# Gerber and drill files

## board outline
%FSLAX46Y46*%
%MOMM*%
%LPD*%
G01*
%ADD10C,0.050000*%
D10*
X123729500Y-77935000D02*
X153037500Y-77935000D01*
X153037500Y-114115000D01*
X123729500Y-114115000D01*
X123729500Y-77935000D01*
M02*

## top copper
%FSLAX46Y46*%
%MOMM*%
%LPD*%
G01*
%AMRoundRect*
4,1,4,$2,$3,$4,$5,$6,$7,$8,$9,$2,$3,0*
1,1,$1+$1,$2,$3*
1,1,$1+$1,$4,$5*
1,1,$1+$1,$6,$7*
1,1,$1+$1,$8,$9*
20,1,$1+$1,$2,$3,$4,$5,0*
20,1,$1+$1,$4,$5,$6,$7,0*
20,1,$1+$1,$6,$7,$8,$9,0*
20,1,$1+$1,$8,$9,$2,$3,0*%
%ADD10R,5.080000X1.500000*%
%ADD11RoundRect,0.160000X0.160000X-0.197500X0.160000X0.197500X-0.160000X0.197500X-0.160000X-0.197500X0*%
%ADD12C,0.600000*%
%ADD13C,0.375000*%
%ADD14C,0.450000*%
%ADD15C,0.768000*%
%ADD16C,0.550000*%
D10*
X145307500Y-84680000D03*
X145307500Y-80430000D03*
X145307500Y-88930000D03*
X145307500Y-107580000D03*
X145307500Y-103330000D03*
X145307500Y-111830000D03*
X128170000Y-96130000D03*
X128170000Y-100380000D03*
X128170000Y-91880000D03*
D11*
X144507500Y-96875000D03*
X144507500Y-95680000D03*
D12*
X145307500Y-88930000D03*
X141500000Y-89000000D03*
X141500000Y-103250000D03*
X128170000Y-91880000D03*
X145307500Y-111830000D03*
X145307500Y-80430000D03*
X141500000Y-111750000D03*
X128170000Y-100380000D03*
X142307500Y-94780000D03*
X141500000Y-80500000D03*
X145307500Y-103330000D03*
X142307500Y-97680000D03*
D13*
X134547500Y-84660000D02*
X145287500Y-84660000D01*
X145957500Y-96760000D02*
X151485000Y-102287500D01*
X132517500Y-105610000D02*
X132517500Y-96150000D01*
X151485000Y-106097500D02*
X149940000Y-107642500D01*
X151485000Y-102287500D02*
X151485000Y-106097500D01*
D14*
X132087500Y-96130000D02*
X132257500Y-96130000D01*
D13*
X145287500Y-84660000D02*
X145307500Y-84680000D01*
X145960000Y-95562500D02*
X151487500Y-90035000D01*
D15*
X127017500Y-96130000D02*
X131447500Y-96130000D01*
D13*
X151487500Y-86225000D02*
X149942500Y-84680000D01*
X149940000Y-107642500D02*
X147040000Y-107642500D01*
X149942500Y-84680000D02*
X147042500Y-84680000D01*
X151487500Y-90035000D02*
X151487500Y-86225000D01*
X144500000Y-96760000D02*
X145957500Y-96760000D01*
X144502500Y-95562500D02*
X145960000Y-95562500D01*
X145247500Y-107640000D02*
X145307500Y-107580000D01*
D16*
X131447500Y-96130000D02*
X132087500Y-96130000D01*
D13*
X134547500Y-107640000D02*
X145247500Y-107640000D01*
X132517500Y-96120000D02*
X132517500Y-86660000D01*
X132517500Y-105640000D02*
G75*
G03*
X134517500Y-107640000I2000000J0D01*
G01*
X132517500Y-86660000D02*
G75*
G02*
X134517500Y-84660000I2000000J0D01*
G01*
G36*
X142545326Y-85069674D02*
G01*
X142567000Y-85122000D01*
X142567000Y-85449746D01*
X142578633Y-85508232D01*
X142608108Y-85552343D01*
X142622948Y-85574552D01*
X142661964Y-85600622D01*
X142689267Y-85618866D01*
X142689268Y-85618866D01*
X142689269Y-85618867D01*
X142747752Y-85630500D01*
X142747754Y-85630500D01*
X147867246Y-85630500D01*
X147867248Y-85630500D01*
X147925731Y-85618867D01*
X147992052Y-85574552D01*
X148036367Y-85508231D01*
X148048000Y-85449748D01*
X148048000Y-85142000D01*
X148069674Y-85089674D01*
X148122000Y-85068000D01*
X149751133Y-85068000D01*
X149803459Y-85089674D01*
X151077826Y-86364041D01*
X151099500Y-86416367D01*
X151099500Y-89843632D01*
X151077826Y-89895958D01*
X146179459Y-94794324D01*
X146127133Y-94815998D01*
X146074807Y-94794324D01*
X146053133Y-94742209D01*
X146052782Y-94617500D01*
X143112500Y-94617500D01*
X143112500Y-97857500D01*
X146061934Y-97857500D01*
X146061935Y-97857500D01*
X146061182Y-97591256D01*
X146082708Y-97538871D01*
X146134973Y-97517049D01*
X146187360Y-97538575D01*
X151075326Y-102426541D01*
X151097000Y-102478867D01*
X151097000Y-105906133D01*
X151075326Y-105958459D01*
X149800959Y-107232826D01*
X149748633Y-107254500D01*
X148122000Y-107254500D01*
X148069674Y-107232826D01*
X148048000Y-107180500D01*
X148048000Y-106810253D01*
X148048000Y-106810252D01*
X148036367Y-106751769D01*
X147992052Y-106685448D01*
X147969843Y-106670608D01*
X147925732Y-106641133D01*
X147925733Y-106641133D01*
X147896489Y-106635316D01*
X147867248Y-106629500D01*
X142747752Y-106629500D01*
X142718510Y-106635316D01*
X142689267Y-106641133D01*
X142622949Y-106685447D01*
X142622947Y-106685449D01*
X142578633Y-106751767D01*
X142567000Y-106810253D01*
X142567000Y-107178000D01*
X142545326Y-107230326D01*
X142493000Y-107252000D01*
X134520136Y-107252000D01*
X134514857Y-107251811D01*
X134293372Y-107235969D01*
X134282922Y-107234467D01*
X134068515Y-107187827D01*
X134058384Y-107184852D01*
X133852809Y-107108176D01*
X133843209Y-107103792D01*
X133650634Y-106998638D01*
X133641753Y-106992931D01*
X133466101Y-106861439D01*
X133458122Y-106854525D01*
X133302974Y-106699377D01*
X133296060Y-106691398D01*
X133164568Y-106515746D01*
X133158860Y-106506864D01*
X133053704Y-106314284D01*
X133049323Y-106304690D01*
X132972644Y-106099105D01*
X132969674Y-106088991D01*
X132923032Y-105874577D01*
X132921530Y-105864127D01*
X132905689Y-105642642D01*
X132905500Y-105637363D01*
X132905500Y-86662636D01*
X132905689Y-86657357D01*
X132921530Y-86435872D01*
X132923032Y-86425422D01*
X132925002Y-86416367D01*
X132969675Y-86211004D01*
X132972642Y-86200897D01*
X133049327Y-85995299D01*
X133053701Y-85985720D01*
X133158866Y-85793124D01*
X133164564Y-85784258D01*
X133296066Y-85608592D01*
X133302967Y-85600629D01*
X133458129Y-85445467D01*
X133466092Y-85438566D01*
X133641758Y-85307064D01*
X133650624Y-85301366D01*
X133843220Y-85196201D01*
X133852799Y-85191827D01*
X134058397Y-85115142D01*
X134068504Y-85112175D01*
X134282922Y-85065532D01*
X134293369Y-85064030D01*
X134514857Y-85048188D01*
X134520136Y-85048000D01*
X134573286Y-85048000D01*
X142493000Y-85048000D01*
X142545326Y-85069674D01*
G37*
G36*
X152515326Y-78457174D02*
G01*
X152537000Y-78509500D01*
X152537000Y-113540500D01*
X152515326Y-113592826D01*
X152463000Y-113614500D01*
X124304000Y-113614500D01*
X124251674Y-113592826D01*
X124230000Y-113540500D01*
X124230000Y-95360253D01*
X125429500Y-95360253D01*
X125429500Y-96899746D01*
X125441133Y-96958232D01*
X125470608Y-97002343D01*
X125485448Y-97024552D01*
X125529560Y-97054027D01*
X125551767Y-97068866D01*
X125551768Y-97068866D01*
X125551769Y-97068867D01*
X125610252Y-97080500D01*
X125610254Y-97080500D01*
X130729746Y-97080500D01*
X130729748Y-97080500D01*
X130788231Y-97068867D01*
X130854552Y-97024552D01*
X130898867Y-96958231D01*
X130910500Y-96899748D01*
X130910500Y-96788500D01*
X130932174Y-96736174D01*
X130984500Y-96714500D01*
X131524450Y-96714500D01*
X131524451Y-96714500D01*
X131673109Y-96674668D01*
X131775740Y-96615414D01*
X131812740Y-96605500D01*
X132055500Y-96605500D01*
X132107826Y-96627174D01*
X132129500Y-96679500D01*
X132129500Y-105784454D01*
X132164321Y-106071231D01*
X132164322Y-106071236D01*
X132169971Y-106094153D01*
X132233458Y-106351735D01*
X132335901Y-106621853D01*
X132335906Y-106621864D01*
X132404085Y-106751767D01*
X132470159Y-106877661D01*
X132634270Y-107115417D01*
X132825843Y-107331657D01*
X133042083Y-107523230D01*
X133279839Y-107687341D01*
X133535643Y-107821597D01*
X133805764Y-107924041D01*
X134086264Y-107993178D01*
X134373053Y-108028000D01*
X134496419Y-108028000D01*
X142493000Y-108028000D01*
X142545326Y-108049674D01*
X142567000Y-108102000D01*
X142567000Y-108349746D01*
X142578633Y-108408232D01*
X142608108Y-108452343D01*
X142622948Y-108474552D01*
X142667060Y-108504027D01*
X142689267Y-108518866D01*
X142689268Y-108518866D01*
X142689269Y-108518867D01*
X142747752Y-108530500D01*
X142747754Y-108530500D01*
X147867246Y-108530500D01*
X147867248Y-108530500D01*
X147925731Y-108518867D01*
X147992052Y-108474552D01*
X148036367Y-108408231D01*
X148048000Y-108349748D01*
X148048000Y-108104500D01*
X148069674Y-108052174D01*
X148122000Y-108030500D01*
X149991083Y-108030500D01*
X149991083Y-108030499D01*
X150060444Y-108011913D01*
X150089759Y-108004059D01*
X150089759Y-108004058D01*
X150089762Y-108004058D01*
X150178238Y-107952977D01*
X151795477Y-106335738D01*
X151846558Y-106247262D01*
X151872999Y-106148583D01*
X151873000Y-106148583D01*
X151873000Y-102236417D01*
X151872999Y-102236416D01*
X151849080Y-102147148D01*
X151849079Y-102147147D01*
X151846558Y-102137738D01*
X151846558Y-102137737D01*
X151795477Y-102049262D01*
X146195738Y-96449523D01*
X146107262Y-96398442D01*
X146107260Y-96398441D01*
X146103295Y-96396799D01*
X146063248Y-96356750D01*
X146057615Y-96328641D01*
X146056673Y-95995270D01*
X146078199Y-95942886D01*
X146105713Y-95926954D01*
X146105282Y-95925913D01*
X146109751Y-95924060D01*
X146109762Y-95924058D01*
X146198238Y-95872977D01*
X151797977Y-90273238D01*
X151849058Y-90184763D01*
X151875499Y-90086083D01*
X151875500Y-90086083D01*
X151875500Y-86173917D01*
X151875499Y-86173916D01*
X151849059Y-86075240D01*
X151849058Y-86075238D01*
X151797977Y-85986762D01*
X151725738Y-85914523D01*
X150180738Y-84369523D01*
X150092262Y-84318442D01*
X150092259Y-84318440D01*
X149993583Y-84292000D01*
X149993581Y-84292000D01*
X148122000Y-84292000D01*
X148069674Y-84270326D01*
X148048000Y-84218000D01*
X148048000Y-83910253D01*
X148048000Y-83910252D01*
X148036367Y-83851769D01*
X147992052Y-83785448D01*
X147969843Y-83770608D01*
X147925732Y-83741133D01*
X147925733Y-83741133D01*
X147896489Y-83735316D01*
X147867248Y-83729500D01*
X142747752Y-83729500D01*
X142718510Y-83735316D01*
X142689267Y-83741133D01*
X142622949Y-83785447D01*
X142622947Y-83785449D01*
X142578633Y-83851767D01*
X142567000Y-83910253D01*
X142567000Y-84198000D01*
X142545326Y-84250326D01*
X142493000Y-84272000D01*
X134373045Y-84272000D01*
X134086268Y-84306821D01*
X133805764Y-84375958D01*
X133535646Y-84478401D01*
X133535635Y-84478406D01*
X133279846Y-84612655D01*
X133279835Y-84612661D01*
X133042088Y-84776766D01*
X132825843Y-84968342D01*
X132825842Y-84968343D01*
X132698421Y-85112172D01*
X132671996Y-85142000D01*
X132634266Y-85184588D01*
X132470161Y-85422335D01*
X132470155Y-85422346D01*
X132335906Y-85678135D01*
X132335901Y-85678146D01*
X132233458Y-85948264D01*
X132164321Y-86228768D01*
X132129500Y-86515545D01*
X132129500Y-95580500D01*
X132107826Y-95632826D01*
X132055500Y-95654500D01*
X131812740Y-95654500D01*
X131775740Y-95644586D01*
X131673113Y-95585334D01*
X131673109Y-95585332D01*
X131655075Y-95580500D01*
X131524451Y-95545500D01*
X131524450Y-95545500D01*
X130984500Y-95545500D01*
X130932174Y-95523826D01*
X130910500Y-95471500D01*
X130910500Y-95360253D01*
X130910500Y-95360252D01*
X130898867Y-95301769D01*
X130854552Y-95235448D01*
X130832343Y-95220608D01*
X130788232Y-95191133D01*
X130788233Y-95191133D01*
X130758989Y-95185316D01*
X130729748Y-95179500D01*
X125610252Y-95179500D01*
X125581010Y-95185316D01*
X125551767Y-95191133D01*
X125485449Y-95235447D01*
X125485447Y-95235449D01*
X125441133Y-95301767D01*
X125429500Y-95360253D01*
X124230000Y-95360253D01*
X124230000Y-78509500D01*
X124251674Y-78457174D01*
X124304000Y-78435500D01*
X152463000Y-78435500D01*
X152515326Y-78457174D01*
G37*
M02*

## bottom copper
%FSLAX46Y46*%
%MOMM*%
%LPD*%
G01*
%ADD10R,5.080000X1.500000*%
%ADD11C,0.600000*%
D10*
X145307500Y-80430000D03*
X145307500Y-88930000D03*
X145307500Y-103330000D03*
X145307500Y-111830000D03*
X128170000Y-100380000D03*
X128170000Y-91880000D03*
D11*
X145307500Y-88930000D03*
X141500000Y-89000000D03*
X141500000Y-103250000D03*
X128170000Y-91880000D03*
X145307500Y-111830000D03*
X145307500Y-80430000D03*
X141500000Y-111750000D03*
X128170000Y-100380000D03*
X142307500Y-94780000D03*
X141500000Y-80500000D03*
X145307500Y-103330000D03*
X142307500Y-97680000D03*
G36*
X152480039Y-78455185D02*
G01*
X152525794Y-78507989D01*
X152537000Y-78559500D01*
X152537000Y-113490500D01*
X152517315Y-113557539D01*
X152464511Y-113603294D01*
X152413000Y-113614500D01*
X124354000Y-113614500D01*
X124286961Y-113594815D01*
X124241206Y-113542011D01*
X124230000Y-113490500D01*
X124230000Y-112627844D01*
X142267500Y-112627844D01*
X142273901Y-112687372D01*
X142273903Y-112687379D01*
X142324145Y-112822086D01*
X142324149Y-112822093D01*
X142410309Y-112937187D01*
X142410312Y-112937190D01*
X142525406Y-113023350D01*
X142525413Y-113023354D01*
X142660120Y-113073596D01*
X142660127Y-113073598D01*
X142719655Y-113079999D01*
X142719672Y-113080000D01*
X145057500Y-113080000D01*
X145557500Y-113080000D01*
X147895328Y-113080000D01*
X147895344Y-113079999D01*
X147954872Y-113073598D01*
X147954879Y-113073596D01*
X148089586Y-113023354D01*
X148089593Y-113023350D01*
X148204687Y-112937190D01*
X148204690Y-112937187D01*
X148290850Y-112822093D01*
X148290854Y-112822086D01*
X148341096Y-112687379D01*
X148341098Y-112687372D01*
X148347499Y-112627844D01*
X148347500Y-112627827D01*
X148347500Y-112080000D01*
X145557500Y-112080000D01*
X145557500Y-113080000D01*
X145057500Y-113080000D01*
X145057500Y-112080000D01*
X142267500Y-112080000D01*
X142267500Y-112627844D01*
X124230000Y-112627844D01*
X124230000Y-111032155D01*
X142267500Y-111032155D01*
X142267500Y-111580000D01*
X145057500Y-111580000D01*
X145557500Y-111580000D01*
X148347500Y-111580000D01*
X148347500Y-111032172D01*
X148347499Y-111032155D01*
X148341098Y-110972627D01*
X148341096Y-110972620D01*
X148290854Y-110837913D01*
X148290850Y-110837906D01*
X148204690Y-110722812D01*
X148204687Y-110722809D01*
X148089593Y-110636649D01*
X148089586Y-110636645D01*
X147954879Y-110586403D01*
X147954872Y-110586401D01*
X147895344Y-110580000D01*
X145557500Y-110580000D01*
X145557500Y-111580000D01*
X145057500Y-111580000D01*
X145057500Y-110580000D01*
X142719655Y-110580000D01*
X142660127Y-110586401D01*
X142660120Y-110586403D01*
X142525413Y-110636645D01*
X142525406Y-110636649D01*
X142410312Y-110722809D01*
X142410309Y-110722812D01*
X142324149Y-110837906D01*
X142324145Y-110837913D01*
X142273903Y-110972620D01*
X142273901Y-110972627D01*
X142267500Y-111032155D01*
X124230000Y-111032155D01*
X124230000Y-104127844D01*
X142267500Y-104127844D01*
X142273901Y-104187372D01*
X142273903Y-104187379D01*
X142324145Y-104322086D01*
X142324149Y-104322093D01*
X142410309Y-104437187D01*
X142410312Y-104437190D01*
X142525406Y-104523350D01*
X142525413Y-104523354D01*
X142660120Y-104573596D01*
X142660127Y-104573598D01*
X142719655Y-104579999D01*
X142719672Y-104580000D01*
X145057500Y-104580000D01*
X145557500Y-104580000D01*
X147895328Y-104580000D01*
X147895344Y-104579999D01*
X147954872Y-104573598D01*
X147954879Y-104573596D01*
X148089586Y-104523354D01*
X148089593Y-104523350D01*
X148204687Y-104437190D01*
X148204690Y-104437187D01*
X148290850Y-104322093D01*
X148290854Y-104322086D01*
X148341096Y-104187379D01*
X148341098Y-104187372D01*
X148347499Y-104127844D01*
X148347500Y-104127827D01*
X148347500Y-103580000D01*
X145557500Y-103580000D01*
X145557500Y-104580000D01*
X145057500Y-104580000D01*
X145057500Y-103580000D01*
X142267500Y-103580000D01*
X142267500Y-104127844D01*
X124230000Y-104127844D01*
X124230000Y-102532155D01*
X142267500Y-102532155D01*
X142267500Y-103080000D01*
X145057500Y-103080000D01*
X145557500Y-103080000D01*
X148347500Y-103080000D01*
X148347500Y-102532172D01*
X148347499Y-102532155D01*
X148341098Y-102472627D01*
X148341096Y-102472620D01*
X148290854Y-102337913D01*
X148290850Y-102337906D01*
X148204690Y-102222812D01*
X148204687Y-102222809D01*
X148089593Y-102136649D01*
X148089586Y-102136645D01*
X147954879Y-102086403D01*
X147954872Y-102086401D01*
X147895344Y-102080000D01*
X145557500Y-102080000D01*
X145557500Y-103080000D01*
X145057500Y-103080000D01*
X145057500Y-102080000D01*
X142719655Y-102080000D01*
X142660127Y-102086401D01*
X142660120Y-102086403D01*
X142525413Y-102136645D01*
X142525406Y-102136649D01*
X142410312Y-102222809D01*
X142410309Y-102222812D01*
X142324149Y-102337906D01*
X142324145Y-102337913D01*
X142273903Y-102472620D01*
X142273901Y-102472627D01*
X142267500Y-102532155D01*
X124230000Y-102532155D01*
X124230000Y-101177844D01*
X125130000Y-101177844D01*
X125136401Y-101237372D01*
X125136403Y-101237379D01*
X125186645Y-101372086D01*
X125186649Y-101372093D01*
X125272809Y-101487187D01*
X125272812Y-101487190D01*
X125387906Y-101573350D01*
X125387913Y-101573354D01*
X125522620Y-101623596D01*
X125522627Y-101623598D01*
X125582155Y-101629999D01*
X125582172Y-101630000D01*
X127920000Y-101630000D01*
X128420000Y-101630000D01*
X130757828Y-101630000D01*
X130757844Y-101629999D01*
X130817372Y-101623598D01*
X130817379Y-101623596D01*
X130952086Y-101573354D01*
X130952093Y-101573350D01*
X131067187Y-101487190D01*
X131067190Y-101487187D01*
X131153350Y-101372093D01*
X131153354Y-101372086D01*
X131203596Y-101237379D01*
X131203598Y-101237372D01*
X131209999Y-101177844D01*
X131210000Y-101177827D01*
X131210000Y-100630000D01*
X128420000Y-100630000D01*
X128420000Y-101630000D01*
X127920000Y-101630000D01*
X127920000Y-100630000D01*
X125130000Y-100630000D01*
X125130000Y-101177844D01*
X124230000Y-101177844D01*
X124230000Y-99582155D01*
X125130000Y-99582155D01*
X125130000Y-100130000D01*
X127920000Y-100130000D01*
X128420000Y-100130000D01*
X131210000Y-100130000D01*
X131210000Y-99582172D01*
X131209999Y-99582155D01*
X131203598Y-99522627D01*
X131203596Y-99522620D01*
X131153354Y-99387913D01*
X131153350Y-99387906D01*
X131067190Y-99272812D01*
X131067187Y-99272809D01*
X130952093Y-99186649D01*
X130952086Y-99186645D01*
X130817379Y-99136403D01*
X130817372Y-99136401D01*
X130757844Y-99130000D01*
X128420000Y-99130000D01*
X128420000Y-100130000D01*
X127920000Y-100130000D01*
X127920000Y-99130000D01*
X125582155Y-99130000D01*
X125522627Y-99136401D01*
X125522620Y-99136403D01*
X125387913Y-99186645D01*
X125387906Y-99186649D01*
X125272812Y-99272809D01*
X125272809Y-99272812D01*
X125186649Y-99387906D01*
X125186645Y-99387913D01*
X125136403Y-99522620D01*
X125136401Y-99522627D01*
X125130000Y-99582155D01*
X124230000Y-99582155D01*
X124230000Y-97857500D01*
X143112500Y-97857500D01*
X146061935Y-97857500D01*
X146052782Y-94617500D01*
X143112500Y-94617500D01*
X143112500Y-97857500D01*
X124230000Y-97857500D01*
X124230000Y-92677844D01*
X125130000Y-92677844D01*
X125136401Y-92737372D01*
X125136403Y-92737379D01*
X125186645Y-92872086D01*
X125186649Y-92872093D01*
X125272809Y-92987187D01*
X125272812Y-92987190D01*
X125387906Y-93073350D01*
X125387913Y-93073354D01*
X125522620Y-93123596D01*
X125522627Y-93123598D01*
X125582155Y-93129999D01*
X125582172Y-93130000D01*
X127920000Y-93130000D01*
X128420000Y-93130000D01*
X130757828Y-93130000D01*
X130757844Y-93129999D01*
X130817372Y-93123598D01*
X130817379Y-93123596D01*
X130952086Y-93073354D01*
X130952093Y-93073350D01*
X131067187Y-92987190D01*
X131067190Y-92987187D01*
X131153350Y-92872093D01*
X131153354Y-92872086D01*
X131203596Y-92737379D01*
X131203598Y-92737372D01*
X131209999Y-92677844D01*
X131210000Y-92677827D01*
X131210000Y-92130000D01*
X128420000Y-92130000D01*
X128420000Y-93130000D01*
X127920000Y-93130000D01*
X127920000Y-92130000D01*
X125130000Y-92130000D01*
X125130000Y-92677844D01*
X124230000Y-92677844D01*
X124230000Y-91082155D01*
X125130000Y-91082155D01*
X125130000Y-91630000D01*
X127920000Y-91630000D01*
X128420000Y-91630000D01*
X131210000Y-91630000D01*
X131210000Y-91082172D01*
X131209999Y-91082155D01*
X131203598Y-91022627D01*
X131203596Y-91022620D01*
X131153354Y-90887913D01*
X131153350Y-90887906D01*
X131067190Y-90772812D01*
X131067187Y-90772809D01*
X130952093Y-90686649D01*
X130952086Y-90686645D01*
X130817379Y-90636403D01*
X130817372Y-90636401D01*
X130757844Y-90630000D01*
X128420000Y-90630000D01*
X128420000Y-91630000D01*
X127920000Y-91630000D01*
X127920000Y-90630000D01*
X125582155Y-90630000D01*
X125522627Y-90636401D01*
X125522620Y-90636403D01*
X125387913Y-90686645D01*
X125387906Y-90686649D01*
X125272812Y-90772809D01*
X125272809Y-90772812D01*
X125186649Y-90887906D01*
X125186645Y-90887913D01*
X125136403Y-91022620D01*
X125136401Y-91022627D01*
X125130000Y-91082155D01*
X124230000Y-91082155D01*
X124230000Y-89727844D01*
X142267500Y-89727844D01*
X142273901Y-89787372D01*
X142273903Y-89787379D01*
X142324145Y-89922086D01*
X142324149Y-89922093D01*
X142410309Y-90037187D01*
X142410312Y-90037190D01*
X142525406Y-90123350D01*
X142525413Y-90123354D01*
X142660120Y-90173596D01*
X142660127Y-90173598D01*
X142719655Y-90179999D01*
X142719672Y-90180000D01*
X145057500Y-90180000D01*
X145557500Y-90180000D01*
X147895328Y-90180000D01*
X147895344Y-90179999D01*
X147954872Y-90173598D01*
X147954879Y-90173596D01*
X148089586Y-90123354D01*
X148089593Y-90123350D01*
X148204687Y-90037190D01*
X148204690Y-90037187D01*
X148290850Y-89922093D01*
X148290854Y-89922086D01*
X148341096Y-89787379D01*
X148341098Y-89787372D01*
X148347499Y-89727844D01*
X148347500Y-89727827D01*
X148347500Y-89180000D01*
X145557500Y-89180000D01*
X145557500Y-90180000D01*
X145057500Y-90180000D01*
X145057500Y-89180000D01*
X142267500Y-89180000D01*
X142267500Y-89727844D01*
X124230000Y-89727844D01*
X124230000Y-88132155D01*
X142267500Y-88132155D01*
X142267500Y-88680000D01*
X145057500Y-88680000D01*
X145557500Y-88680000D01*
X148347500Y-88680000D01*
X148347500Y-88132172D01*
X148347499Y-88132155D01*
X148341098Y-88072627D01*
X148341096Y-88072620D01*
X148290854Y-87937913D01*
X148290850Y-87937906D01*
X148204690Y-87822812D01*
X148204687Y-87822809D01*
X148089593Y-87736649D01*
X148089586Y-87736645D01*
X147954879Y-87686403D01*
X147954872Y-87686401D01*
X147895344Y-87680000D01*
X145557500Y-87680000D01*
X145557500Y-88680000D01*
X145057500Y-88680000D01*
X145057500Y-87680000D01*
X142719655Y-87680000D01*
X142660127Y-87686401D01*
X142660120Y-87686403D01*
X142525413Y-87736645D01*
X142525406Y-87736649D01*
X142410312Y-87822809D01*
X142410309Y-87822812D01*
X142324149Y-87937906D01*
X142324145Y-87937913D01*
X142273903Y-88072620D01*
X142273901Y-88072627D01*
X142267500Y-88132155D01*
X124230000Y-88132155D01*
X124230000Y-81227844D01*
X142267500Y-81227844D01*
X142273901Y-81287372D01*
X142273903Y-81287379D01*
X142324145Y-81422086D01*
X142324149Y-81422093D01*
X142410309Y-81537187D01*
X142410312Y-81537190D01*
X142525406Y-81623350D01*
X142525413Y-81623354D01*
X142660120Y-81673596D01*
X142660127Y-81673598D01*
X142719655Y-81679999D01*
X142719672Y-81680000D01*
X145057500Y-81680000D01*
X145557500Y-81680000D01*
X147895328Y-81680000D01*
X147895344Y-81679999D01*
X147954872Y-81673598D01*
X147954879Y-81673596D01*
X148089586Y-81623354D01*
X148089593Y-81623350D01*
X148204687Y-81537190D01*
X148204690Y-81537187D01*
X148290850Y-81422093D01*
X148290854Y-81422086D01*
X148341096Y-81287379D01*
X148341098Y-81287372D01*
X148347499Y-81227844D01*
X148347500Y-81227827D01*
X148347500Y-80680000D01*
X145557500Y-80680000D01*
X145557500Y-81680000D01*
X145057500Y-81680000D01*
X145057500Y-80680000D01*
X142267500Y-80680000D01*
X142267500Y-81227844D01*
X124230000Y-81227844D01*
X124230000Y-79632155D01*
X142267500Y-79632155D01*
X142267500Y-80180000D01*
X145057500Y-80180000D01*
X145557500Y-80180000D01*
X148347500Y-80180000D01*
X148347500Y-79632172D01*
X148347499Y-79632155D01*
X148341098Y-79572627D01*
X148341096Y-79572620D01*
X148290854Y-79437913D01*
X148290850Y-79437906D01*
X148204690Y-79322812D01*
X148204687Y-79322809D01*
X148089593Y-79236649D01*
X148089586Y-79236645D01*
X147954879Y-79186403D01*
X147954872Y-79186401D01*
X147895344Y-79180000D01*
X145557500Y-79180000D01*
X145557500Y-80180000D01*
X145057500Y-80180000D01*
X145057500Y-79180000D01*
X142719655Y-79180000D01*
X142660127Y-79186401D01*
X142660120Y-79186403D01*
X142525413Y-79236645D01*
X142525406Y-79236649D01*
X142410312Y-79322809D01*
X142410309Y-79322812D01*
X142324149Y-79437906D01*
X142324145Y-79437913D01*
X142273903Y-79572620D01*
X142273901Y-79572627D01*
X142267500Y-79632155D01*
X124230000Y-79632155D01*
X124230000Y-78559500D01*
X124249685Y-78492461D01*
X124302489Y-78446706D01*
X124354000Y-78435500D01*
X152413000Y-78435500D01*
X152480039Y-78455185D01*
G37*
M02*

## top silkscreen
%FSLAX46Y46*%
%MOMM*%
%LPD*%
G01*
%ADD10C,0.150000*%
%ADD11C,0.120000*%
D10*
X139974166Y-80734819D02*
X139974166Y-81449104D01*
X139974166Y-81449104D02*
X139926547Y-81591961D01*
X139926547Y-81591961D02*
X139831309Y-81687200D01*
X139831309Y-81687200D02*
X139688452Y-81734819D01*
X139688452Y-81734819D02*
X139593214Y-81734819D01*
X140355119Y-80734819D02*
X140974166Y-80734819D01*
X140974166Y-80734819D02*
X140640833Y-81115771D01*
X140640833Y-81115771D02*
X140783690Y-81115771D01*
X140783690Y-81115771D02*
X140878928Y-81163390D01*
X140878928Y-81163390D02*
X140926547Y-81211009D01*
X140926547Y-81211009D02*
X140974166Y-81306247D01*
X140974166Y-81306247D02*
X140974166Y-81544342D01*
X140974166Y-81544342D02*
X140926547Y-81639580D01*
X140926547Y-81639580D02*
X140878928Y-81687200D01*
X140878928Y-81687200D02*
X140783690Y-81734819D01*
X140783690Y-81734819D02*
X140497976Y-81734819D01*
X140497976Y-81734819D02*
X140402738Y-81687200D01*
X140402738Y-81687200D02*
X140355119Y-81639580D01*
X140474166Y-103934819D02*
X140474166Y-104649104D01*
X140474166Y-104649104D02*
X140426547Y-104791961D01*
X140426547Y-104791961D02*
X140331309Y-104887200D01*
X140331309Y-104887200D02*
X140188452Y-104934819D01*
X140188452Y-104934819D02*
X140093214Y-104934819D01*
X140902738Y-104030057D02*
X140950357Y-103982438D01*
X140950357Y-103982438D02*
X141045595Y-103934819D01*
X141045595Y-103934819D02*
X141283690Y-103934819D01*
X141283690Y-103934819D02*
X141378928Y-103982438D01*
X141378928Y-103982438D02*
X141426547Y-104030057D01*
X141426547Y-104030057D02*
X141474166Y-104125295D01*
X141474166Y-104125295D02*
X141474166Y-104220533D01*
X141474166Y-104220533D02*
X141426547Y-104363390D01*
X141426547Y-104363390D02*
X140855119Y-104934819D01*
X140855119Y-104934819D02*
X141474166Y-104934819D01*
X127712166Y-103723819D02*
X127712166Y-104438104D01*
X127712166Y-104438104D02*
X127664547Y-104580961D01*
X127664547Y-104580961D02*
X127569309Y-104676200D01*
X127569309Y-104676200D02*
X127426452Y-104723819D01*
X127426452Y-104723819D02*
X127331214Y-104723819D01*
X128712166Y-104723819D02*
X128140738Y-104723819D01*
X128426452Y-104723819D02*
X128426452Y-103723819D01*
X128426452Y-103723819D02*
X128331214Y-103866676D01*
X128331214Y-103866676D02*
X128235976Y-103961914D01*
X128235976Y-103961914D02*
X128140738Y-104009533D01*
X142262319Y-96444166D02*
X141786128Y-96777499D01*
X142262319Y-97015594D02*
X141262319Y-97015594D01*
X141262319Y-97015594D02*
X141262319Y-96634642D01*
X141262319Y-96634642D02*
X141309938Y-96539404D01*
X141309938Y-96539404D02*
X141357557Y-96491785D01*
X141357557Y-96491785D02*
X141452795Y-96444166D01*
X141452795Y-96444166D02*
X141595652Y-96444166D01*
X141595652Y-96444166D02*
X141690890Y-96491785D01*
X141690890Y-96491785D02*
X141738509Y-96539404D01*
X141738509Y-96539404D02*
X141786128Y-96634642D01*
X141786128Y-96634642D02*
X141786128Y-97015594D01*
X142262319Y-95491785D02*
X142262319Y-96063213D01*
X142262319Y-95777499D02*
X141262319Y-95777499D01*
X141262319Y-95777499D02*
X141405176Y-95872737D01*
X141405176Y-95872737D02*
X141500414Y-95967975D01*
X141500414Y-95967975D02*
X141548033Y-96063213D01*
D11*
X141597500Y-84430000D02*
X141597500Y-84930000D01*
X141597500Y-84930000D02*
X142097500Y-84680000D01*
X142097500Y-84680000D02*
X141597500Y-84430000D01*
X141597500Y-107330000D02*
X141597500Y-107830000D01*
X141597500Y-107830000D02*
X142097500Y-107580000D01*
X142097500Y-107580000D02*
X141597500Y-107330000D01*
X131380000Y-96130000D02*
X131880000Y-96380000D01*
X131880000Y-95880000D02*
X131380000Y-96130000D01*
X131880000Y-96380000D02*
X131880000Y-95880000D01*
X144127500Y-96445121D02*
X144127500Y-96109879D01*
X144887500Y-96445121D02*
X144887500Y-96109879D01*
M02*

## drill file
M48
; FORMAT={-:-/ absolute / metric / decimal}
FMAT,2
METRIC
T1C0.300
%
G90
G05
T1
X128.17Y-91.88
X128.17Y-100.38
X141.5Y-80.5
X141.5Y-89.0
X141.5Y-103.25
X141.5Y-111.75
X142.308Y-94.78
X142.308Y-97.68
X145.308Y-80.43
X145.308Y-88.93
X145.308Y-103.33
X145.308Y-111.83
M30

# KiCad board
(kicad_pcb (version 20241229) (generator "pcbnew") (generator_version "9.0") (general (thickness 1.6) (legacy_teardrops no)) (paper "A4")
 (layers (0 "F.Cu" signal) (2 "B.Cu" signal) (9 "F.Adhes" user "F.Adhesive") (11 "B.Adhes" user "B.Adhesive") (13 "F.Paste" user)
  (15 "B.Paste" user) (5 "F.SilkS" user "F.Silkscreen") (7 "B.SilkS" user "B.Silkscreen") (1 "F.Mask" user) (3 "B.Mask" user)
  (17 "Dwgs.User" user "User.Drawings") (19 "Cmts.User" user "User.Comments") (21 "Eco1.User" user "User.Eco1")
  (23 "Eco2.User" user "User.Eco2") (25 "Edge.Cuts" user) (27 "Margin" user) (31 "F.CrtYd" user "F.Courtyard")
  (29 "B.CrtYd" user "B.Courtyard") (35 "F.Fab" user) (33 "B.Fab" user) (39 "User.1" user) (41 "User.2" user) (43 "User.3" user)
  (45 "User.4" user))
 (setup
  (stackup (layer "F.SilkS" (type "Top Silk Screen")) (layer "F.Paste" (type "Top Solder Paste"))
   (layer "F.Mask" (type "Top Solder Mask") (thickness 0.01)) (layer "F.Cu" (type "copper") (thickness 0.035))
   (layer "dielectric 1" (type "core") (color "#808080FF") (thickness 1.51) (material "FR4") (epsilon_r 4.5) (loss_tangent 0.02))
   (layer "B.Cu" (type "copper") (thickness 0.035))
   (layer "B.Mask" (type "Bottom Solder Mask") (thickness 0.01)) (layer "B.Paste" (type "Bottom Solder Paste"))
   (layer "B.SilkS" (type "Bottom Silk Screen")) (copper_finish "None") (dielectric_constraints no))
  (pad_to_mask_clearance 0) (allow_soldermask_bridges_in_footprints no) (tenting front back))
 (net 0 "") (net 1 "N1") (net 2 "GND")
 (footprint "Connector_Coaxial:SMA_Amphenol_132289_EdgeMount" (layer "F.Cu") (at 145.3075 84.68)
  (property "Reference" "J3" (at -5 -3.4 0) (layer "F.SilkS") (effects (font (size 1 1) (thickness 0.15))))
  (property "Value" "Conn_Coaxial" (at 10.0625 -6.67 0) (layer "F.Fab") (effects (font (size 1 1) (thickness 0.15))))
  (fp_line (start -3.71 -0.25) (end -3.71 0.25) (stroke (width 0.12) (type solid)) (layer "F.SilkS"))
  (fp_line (start -3.71 0.25) (end -3.21 0) (stroke (width 0.12) (type solid)) (layer "F.SilkS"))
  (fp_line (start -3.21 0) (end -3.71 -0.25) (stroke (width 0.12) (type solid)) (layer "F.SilkS"))
  (pad "1" smd rect (at 0 0 90) (size 1.5 5.08) (layers "F.Cu" "F.Mask" "F.Paste") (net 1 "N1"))
  (pad "2" smd rect (at 0 -4.25 90) (size 1.5 5.08) (layers "F.Cu" "F.Mask" "F.Paste") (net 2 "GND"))
  (pad "2" smd rect (at 0 -4.25 90) (size 1.5 5.08) (layers "B.Cu" "B.Mask" "B.Paste") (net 2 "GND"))
  (pad "2" smd rect (at 0 4.25 90) (size 1.5 5.08) (layers "F.Cu" "F.Mask" "F.Paste") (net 2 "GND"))
  (pad "2" smd rect (at 0 4.25 90) (size 1.5 5.08) (layers "B.Cu" "B.Mask" "B.Paste") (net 2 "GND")))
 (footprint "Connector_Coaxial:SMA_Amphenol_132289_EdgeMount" (layer "F.Cu") (at 145.3075 107.58)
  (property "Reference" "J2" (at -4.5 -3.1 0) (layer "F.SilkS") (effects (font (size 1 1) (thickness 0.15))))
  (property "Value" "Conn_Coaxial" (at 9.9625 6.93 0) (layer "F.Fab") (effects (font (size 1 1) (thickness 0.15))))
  (fp_line (start -3.71 -0.25) (end -3.71 0.25) (stroke (width 0.12) (type solid)) (layer "F.SilkS"))
  (fp_line (start -3.71 0.25) (end -3.21 0) (stroke (width 0.12) (type solid)) (layer "F.SilkS"))
  (fp_line (start -3.21 0) (end -3.71 -0.25) (stroke (width 0.12) (type solid)) (layer "F.SilkS"))
  (pad "1" smd rect (at 0 0 90) (size 1.5 5.08) (layers "F.Cu" "F.Mask" "F.Paste") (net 1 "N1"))
  (pad "2" smd rect (at 0 -4.25 90) (size 1.5 5.08) (layers "F.Cu" "F.Mask" "F.Paste") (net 2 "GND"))
  (pad "2" smd rect (at 0 -4.25 90) (size 1.5 5.08) (layers "B.Cu" "B.Mask" "B.Paste") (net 2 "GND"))
  (pad "2" smd rect (at 0 4.25 90) (size 1.5 5.08) (layers "F.Cu" "F.Mask" "F.Paste") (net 2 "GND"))
  (pad "2" smd rect (at 0 4.25 90) (size 1.5 5.08) (layers "B.Cu" "B.Mask" "B.Paste") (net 2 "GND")))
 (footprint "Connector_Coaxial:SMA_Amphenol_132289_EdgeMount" (layer "F.Cu") (at 128.17 96.13 180)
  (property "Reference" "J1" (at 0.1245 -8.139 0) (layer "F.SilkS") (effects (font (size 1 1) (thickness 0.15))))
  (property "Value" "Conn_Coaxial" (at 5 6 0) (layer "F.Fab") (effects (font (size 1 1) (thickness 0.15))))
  (fp_line (start -3.21 0) (end -3.71 -0.25) (stroke (width 0.12) (type solid)) (layer "F.SilkS"))
  (fp_line (start -3.71 0.25) (end -3.21 0) (stroke (width 0.12) (type solid)) (layer "F.SilkS"))
  (fp_line (start -3.71 -0.25) (end -3.71 0.25) (stroke (width 0.12) (type solid)) (layer "F.SilkS"))
  (pad "1" smd rect (at 0 0 270) (size 1.5 5.08) (layers "F.Cu" "F.Mask" "F.Paste") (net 1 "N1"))
  (pad "2" smd rect (at 0 -4.25 270) (size 1.5 5.08) (layers "F.Cu" "F.Mask" "F.Paste") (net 2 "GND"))
  (pad "2" smd rect (at 0 -4.25 270) (size 1.5 5.08) (layers "B.Cu" "B.Mask" "B.Paste") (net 2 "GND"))
  (pad "2" smd rect (at 0 4.25 270) (size 1.5 5.08) (layers "F.Cu" "F.Mask" "F.Paste") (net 2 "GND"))
  (pad "2" smd rect (at 0 4.25 270) (size 1.5 5.08) (layers "B.Cu" "B.Mask" "B.Paste") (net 2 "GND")))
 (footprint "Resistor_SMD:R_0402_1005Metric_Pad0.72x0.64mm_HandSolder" (layer "F.Cu") (at 144.5075 96.2775 90)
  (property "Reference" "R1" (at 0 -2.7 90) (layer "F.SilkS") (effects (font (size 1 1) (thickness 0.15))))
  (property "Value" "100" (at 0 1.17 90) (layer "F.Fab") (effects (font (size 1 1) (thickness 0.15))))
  (fp_line (start -0.167621 -0.38) (end 0.167621 -0.38) (stroke (width 0.12) (type solid)) (layer "F.SilkS"))
  (fp_line (start -0.167621 0.38) (end 0.167621 0.38) (stroke (width 0.12) (type solid)) (layer "F.SilkS"))
  (pad "1" smd roundrect (at -0.5975 0 90) (size 0.715 0.64) (layers "F.Cu" "F.Mask" "F.Paste") (roundrect_rratio 0.25) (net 1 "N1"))
  (pad "2" smd roundrect (at 0.5975 0 90) (size 0.715 0.64) (layers "F.Cu" "F.Mask" "F.Paste") (roundrect_rratio 0.25) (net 1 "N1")))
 (gr_rect (start 123.7295 77.935) (end 153.0375 114.115) (stroke (width 0.05) (type default)) (fill no) (layer "Edge.Cuts"))
 (via (at 145.3075 88.93) (size 0.6) (drill 0.3) (layers "F.Cu" "B.Cu") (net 2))
 (via (at 141.5 89) (size 0.6) (drill 0.3) (layers "F.Cu" "B.Cu") (free yes) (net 2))
 (via (at 141.5 103.25) (size 0.6) (drill 0.3) (layers "F.Cu" "B.Cu") (free yes) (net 2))
 (via (at 128.17 91.88) (size 0.6) (drill 0.3) (layers "F.Cu" "B.Cu") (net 2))
 (via (at 145.3075 111.83) (size 0.6) (drill 0.3) (layers "F.Cu" "B.Cu") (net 2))
 (via (at 145.3075 80.43) (size 0.6) (drill 0.3) (layers "F.Cu" "B.Cu") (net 2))
 (via (at 141.5 111.75) (size 0.6) (drill 0.3) (layers "F.Cu" "B.Cu") (free yes) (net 2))
 (via (at 128.17 100.38) (size 0.6) (drill 0.3) (layers "F.Cu" "B.Cu") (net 2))
 (via (at 142.3075 94.78) (size 0.6) (drill 0.3) (layers "F.Cu" "B.Cu") (free yes) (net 2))
 (via (at 141.5 80.5) (size 0.6) (drill 0.3) (layers "F.Cu" "B.Cu") (free yes) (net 2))
 (via (at 145.3075 103.33) (size 0.6) (drill 0.3) (layers "F.Cu" "B.Cu") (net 2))
 (via (at 142.3075 97.68) (size 0.6) (drill 0.3) (layers "F.Cu" "B.Cu") (free yes) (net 2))
 (segment (start 134.5475 84.66) (end 145.2875 84.66) (width 0.375) (layer "F.Cu") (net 1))
 (segment (start 145.9575 96.76) (end 151.485 102.2875) (width 0.375) (layer "F.Cu") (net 1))
 (segment (start 132.5175 105.61) (end 132.5175 96.15) (width 0.375) (layer "F.Cu") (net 1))
 (segment (start 151.485 106.0975) (end 149.94 107.6425) (width 0.375) (layer "F.Cu") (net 1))
 (segment (start 151.485 102.2875) (end 151.485 106.0975) (width 0.375) (layer "F.Cu") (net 1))
 (segment (start 132.0875 96.13) (end 132.2575 96.13) (width 0.45) (layer "F.Cu") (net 1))
 (segment (start 145.2875 84.66) (end 145.3075 84.68) (width 0.375) (layer "F.Cu") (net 1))
 (segment (start 145.96 95.5625) (end 151.4875 90.035) (width 0.375) (layer "F.Cu") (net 1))
 (segment (start 127.0175 96.13) (end 131.4475 96.13) (width 0.768) (layer "F.Cu") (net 1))
 (segment (start 151.4875 86.225) (end 149.9425 84.68) (width 0.375) (layer "F.Cu") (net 1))
 (segment (start 149.94 107.6425) (end 147.04 107.6425) (width 0.375) (layer "F.Cu") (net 1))
 (segment (start 149.9425 84.68) (end 147.0425 84.68) (width 0.375) (layer "F.Cu") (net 1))
 (segment (start 151.4875 90.035) (end 151.4875 86.225) (width 0.375) (layer "F.Cu") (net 1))
 (segment (start 144.5 96.76) (end 145.9575 96.76) (width 0.375) (layer "F.Cu") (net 1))
 (segment (start 144.5025 95.5625) (end 145.96 95.5625) (width 0.375) (layer "F.Cu") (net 1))
 (segment (start 145.2475 107.64) (end 145.3075 107.58) (width 0.375) (layer "F.Cu") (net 1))
 (segment (start 131.4475 96.13) (end 132.0875 96.13) (width 0.55) (layer "F.Cu") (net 1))
 (segment (start 134.5475 107.64) (end 145.2475 107.64) (width 0.375) (layer "F.Cu") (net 1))
 (segment (start 132.5175 96.12) (end 132.5175 86.66) (width 0.375) (layer "F.Cu") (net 1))
 (arc (start 132.5175 105.64) (mid 133.103286 107.054213) (end 134.5175 107.64) (width 0.375) (layer "F.Cu") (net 1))
 (arc (start 132.5175 86.66) (mid 133.103286 85.245787) (end 134.5175 84.66) (width 0.375) (layer "F.Cu") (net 1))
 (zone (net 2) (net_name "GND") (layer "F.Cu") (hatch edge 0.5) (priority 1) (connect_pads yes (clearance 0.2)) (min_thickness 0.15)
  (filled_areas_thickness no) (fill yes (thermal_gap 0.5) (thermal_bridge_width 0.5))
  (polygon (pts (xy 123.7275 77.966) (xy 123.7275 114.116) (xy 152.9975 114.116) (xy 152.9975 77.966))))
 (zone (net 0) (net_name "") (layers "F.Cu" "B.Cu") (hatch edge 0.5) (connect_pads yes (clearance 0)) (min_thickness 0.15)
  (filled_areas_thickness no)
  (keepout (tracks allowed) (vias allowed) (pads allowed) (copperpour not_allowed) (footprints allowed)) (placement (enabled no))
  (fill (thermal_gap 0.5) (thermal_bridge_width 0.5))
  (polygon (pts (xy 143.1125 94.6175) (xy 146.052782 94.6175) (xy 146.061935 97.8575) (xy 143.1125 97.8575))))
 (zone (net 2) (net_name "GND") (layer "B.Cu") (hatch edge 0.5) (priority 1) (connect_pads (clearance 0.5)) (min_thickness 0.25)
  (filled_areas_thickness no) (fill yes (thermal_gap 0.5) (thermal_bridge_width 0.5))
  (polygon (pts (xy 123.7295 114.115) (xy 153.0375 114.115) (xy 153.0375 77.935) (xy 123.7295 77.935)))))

